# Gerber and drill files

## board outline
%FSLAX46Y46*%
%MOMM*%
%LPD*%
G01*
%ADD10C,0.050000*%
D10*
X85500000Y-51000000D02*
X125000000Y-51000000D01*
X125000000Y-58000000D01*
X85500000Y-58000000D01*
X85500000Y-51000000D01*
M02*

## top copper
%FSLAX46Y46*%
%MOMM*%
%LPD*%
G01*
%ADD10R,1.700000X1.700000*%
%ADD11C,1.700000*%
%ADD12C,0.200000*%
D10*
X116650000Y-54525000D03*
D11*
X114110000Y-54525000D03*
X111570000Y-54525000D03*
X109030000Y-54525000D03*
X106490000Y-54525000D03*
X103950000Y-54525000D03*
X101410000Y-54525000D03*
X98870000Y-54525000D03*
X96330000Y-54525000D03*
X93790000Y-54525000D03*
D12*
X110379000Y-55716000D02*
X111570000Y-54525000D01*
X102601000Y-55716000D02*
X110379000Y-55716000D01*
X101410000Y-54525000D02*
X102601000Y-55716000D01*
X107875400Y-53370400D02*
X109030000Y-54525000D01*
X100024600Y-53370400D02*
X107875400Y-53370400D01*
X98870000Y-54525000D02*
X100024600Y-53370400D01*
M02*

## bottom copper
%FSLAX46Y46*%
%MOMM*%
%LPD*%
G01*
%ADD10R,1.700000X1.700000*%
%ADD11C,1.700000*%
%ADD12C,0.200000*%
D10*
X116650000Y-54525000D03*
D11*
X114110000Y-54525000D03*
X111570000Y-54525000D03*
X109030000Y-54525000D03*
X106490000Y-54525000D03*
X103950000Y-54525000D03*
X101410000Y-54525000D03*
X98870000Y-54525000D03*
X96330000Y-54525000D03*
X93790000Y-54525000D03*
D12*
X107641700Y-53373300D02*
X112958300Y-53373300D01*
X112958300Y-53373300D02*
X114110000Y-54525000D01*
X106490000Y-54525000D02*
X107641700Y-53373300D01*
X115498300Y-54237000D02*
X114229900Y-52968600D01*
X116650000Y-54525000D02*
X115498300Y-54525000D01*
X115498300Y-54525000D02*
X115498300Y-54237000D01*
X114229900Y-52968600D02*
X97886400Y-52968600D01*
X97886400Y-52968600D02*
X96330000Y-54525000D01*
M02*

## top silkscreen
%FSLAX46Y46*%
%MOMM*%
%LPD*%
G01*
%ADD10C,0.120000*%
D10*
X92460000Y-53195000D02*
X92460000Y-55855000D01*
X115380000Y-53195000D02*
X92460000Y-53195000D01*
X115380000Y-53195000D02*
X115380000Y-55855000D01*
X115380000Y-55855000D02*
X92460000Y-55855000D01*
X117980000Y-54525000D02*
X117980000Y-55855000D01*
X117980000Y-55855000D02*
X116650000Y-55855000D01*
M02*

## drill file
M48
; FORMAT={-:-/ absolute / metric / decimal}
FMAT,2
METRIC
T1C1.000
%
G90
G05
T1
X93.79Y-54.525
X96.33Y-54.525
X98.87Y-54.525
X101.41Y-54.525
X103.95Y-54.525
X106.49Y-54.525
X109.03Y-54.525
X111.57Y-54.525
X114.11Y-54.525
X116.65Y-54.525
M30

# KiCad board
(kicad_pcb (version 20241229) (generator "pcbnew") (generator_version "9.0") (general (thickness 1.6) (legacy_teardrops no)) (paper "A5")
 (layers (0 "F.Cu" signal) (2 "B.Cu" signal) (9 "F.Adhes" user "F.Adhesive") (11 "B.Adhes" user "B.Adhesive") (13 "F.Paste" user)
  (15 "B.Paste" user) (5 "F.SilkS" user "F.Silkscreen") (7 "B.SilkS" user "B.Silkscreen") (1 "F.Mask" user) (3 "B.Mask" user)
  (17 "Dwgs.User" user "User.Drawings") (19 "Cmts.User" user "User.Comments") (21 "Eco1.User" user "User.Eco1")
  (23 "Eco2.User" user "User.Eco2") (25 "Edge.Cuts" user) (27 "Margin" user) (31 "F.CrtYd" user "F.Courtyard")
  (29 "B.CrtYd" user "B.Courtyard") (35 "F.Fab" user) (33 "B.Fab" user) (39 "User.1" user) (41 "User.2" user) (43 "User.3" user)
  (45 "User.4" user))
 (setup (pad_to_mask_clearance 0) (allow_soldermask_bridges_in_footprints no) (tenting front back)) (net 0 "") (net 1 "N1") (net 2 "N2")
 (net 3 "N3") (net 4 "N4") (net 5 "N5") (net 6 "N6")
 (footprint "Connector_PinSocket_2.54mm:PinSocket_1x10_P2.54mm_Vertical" (layer "F.Cu") (at 116.65 54.525 -90)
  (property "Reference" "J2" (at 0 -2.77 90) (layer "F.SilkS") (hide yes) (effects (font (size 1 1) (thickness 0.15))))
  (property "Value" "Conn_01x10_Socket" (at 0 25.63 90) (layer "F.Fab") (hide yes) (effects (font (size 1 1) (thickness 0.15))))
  (fp_line (start -1.33 24.19) (end 1.33 24.19) (stroke (width 0.12) (type solid)) (layer "F.SilkS"))
  (fp_line (start -1.33 1.27) (end -1.33 24.19) (stroke (width 0.12) (type solid)) (layer "F.SilkS"))
  (fp_line (start -1.33 1.27) (end 1.33 1.27) (stroke (width 0.12) (type solid)) (layer "F.SilkS"))
  (fp_line (start 1.33 1.27) (end 1.33 24.19) (stroke (width 0.12) (type solid)) (layer "F.SilkS"))
  (fp_line (start 0 -1.33) (end 1.33 -1.33) (stroke (width 0.12) (type solid)) (layer "F.SilkS"))
  (fp_line (start 1.33 -1.33) (end 1.33 0) (stroke (width 0.12) (type solid)) (layer "F.SilkS"))
  (pad "5" thru_hole rect (at 0 0 270) (size 1.7 1.7) (drill 1) (layers "*.Cu" "*.Mask") (remove_unused_layers no) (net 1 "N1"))
  (pad "6" thru_hole circle (at 0 2.54 270) (size 1.7 1.7) (drill 1) (layers "*.Cu" "*.Mask") (remove_unused_layers no) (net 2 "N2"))
  (pad "7" thru_hole circle (at 0 5.08 270) (size 1.7 1.7) (drill 1) (layers "*.Cu" "*.Mask") (remove_unused_layers no) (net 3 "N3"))
  (pad "8" thru_hole circle (at 0 7.62 270) (size 1.7 1.7) (drill 1) (layers "*.Cu" "*.Mask") (remove_unused_layers no) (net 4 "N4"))
  (pad "9" thru_hole circle (at 0 10.16 270) (size 1.7 1.7) (drill 1) (layers "*.Cu" "*.Mask") (remove_unused_layers no) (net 2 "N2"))
  (pad "10" thru_hole circle (at 0 12.7 270) (size 1.7 1.7) (drill 1) (layers "*.Cu" "*.Mask") (remove_unused_layers no) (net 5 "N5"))
  (pad "11" thru_hole circle (at 0 15.24 270) (size 1.7 1.7) (drill 1) (layers "*.Cu" "*.Mask") (remove_unused_layers no) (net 3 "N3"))
  (pad "12" thru_hole circle (at 0 17.78 270) (size 1.7 1.7) (drill 1) (layers "*.Cu" "*.Mask") (remove_unused_layers no) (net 4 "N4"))
  (pad "13" thru_hole circle (at 0 20.32 270) (size 1.7 1.7) (drill 1) (layers "*.Cu" "*.Mask") (remove_unused_layers no) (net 1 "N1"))
  (pad "14" thru_hole circle (at 0 22.86 270) (size 1.7 1.7) (drill 1) (layers "*.Cu" "*.Mask") (remove_unused_layers no) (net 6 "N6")))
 (gr_rect (start 85.5 51) (end 125 58) (stroke (width 0.05) (type default)) (fill no) (layer "Edge.Cuts"))
 (segment (start 110.379 55.716) (end 111.57 54.525) (width 0.2) (layer "F.Cu") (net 3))
 (segment (start 102.601 55.716) (end 110.379 55.716) (width 0.2) (layer "F.Cu") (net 3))
 (segment (start 101.41 54.525) (end 102.601 55.716) (width 0.2) (layer "F.Cu") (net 3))
 (segment (start 107.8754 53.3704) (end 109.03 54.525) (width 0.2) (layer "F.Cu") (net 4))
 (segment (start 100.0246 53.3704) (end 107.8754 53.3704) (width 0.2) (layer "F.Cu") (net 4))
 (segment (start 98.87 54.525) (end 100.0246 53.3704) (width 0.2) (layer "F.Cu") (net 4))
 (segment (start 107.6417 53.3733) (end 112.9583 53.3733) (width 0.2) (layer "B.Cu") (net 2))
 (segment (start 112.9583 53.3733) (end 114.11 54.525) (width 0.2) (layer "B.Cu") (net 2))
 (segment (start 106.49 54.525) (end 107.6417 53.3733) (width 0.2) (layer "B.Cu") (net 2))
 (segment (start 115.4983 54.237) (end 114.2299 52.9686) (width 0.2) (layer "B.Cu") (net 1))
 (segment (start 116.65 54.525) (end 115.4983 54.525) (width 0.2) (layer "B.Cu") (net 1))
 (segment (start 115.4983 54.525) (end 115.4983 54.237) (width 0.2) (layer "B.Cu") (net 1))
 (segment (start 114.2299 52.9686) (end 97.8864 52.9686) (width 0.2) (layer "B.Cu") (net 1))
 (segment (start 97.8864 52.9686) (end 96.33 54.525) (width 0.2) (layer "B.Cu") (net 1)))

